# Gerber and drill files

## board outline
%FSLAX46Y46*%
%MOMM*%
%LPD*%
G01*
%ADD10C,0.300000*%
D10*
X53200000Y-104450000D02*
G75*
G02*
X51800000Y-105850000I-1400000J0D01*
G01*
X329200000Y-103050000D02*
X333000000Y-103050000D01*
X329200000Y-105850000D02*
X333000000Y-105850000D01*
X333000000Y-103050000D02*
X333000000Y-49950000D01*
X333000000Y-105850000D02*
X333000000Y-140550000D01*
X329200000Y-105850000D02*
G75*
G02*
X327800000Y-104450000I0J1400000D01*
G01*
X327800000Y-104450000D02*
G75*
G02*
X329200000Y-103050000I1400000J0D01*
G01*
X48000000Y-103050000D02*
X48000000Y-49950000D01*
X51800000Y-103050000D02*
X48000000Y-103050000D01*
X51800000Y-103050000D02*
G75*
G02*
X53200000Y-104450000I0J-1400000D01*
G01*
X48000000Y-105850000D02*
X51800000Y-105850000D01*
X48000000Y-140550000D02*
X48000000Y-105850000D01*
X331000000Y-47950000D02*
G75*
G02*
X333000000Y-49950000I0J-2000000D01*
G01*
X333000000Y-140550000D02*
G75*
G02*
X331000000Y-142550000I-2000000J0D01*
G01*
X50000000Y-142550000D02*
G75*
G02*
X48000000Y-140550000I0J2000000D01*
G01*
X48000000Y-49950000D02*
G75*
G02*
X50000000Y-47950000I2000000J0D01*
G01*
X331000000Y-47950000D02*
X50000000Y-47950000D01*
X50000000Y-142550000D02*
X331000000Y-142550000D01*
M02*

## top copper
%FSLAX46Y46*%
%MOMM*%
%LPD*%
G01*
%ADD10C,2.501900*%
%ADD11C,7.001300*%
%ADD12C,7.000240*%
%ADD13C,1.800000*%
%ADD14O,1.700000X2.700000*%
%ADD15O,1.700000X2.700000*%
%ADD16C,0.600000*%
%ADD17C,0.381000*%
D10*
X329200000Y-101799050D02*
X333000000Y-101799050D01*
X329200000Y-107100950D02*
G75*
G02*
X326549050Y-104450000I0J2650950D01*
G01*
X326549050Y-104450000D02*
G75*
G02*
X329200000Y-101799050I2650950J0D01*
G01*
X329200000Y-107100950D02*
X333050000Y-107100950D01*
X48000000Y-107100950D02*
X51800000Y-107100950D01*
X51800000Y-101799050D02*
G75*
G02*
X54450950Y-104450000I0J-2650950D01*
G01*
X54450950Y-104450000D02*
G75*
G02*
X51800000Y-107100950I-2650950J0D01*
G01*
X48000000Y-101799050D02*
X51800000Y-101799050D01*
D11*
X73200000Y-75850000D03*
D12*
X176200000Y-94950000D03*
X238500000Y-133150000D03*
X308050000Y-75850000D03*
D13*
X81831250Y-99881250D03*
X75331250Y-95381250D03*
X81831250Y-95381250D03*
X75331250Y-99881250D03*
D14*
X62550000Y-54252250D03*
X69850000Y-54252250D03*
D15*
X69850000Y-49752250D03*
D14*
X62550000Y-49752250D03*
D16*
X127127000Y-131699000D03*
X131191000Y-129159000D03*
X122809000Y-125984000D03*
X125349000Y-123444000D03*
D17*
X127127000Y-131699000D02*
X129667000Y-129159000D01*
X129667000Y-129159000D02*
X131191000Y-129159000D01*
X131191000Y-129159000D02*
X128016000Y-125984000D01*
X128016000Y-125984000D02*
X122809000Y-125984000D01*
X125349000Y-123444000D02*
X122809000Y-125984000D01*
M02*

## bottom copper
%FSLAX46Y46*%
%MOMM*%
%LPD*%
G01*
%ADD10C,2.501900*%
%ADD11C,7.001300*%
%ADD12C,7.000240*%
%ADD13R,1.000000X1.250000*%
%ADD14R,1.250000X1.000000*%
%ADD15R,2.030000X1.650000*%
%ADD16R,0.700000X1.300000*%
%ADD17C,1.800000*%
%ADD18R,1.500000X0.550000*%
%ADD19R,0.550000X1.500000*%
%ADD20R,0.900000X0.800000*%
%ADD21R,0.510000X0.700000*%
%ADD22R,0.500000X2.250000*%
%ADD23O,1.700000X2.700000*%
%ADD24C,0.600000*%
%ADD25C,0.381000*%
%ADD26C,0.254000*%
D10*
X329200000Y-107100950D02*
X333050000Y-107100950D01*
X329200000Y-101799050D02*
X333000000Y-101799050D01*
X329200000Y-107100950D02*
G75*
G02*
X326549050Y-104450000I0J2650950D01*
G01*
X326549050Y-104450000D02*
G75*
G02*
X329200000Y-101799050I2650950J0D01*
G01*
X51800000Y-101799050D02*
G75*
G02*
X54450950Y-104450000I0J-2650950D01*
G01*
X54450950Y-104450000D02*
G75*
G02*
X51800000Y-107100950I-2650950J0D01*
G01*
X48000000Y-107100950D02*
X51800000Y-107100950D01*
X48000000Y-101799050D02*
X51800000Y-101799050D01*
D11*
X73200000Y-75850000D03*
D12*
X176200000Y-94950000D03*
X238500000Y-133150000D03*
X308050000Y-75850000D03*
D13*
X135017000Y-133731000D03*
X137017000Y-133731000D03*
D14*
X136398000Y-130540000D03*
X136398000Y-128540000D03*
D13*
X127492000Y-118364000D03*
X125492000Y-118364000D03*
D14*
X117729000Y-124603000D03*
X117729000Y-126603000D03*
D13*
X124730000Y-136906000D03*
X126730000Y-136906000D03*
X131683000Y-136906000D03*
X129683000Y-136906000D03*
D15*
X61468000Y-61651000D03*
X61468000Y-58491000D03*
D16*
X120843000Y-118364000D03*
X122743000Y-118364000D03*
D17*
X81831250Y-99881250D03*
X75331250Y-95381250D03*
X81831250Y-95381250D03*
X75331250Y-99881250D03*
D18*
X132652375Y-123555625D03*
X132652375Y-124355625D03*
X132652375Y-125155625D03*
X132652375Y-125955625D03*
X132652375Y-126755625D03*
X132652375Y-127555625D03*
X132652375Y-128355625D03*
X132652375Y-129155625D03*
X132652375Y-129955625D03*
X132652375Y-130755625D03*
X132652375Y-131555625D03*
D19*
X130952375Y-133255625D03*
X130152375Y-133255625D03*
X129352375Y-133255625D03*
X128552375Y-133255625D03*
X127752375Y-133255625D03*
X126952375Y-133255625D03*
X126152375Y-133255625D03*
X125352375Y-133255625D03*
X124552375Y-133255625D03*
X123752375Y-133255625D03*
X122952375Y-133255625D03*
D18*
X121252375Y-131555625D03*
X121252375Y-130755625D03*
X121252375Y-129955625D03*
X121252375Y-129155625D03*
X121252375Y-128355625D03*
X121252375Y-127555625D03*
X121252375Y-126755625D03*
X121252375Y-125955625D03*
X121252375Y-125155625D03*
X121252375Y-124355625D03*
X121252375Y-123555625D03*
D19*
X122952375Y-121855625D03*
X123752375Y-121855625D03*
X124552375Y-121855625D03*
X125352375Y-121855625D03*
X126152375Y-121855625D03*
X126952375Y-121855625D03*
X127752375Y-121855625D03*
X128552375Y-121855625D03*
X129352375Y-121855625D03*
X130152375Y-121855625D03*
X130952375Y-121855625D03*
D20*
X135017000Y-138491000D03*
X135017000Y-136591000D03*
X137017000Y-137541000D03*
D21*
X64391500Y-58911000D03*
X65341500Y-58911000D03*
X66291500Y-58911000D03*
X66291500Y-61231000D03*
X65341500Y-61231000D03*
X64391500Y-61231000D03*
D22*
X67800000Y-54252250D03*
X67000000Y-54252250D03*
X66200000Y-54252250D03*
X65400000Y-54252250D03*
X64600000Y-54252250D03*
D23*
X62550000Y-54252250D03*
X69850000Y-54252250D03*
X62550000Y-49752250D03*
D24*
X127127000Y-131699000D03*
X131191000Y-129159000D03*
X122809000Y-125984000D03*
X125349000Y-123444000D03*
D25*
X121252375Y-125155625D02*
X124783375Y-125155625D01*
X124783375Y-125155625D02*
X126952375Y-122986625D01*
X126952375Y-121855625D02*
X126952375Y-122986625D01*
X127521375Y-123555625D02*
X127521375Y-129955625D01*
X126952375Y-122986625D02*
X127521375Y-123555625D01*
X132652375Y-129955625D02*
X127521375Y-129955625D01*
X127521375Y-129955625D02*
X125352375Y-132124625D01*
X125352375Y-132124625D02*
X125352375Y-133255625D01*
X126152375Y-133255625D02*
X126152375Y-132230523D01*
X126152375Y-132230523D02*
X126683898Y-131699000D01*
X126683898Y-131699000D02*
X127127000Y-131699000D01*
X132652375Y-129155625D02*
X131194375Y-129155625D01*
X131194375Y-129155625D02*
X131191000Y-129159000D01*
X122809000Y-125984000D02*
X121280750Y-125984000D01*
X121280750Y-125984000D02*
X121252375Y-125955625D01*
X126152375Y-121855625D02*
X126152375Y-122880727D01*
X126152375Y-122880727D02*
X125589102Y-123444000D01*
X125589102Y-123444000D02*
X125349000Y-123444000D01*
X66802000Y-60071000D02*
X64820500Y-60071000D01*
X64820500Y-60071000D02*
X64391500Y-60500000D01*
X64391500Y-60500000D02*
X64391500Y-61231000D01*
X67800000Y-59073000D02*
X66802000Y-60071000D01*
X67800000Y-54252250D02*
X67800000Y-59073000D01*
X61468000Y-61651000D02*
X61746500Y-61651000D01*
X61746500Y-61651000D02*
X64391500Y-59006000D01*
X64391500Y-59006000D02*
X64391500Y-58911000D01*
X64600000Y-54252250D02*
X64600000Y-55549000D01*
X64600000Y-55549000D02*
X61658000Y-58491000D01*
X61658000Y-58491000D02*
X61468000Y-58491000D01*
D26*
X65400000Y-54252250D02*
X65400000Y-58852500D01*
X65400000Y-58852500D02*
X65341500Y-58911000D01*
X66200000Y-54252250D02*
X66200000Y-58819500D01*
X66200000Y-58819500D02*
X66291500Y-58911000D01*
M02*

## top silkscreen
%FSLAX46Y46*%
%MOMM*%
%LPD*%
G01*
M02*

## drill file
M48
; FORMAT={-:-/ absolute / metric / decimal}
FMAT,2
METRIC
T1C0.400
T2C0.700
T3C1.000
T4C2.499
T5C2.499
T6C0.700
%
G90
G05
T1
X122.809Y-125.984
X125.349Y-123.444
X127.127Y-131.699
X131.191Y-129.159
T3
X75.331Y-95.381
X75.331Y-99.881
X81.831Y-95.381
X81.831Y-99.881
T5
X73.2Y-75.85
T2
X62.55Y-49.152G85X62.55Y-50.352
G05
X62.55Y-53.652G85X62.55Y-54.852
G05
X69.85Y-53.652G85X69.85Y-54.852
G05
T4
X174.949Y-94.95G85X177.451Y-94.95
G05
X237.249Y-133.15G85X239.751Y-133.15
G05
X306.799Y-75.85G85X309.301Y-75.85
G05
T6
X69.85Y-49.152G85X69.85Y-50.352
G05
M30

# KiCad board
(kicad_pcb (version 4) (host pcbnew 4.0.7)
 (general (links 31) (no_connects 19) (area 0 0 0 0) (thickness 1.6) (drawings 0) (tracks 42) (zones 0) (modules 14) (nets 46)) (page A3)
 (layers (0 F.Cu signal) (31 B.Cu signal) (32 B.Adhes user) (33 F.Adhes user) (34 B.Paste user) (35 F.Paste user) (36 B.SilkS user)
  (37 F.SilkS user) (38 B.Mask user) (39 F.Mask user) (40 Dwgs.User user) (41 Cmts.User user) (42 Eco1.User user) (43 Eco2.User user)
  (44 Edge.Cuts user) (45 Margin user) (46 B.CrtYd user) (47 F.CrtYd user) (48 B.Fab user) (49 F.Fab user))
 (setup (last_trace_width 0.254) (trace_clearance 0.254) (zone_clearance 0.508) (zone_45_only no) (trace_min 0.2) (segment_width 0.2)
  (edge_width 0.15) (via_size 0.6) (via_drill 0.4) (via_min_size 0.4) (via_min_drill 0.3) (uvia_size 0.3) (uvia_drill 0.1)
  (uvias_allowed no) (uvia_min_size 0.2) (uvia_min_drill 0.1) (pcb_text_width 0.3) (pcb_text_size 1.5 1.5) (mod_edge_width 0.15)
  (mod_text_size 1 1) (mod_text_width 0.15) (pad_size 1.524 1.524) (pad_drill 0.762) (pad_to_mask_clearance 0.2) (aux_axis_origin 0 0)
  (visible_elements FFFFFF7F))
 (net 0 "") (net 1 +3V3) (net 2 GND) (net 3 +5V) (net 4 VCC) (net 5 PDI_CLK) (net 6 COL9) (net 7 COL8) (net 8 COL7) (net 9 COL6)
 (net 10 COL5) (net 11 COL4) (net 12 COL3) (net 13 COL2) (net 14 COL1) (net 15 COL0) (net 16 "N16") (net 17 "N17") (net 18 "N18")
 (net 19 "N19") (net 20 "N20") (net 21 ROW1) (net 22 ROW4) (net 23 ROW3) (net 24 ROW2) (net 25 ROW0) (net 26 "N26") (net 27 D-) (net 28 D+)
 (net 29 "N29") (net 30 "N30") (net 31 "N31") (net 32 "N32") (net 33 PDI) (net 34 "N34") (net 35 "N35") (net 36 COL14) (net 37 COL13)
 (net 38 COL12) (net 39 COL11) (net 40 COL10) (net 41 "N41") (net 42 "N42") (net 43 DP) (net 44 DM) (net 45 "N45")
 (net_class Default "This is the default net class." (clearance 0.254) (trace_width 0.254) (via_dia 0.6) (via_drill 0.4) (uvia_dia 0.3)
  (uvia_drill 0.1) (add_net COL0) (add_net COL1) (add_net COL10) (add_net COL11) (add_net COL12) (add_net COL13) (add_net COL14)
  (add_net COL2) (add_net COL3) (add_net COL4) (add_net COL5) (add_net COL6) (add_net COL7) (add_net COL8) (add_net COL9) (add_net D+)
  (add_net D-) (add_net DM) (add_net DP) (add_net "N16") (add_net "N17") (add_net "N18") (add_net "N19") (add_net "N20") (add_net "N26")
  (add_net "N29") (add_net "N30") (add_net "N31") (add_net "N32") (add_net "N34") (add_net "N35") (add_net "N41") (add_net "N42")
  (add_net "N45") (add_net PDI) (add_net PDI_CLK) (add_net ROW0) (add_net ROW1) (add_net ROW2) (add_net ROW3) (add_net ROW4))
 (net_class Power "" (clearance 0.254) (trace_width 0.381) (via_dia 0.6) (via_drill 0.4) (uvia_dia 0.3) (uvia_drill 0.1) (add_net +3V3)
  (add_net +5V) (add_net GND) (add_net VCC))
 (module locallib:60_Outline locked (layer F.Cu) (at 190.5 95.25)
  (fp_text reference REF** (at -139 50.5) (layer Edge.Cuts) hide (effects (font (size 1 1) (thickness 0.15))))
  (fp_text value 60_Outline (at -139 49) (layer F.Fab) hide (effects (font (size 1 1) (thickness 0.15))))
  (fp_line (start 138.7 11.85095) (end 142.55 11.85095) (layer B.Cu) (width 2.5019))
  (fp_line (start 138.7 6.54905) (end 142.5 6.54905) (layer F.Cu) (width 2.5019))
  (fp_arc (start 138.7 9.2) (end 136.04905 9.2) (angle -90) (layer F.Cu) (width 2.5019))
  (fp_arc (start 138.7 9.2) (end 138.7 6.54905) (angle -90) (layer F.Cu) (width 2.5019))
  (fp_line (start 138.7 6.54905) (end 142.5 6.54905) (layer B.Cu) (width 2.5019))
  (fp_line (start 138.7 11.85095) (end 142.55 11.85095) (layer F.Cu) (width 2.5019))
  (fp_arc (start 138.7 9.2) (end 136.04905 9.2) (angle -90) (layer B.Cu) (width 2.5019))
  (fp_arc (start 138.7 9.2) (end 138.7 6.54905) (angle -90) (layer B.Cu) (width 2.5019))
  (fp_arc (start -138.7 9.2) (end -138.7 6.54905) (angle 90) (layer B.Cu) (width 2.5019))
  (fp_arc (start -138.7 9.2) (end -136.04905 9.2) (angle 90) (layer B.Cu) (width 2.5019))
  (fp_line (start -142.5 11.85095) (end -138.7 11.85095) (layer F.Cu) (width 2.5019))
  (fp_line (start -142.5 11.85095) (end -138.7 11.85095) (layer B.Cu) (width 2.5019))
  (fp_arc (start -138.7 9.2) (end -138.7 6.54905) (angle 90) (layer F.Cu) (width 2.5019))
  (fp_arc (start -138.7 9.2) (end -136.04905 9.2) (angle 90) (layer F.Cu) (width 2.5019))
  (fp_arc (start -138.7 9.2) (end -137.3 9.2) (angle 90) (layer Edge.Cuts) (width 0.3))
  (fp_line (start -142.5 6.54905) (end -138.7 6.54905) (layer B.Cu) (width 2.5019))
  (fp_line (start -142.5 6.54905) (end -138.7 6.54905) (layer F.Cu) (width 2.5019))
  (fp_line (start 138.7 7.8) (end 142.5 7.8) (layer Edge.Cuts) (width 0.3))
  (fp_line (start 138.7 10.6) (end 142.5 10.6) (layer Edge.Cuts) (width 0.3))
  (fp_line (start 142.5 7.8) (end 142.5 -45.3) (layer Edge.Cuts) (width 0.3))
  (fp_line (start 142.5 10.6) (end 142.5 45.3) (layer Edge.Cuts) (width 0.3))
  (fp_arc (start 138.7 9.2) (end 137.3 9.2) (angle -90) (layer Edge.Cuts) (width 0.3))
  (fp_arc (start 138.7 9.2) (end 138.7 7.8) (angle -90) (layer Edge.Cuts) (width 0.3))
  (fp_line (start -142.5 7.8) (end -142.5 -45.3) (layer Edge.Cuts) (width 0.3))
  (fp_line (start -138.7 7.8) (end -142.5 7.8) (layer Edge.Cuts) (width 0.3))
  (fp_arc (start -138.7 9.2) (end -138.7 7.8) (angle 90) (layer Edge.Cuts) (width 0.3))
  (fp_line (start -142.5 10.6) (end -138.7 10.6) (layer Edge.Cuts) (width 0.3))
  (fp_line (start -142.5 45.3) (end -142.5 10.6) (layer Edge.Cuts) (width 0.3))
  (fp_arc (start 140.5 -45.3) (end 140.5 -47.3) (angle 90) (layer Edge.Cuts) (width 0.3))
  (fp_arc (start 140.5 45.3) (end 142.5 45.3) (angle 90) (layer Edge.Cuts) (width 0.3))
  (fp_arc (start -140.5 45.3) (end -140.5 47.3) (angle 90) (layer Edge.Cuts) (width 0.3))
  (fp_arc (start -140.5 -45.3) (end -142.5 -45.3) (angle 90) (layer Edge.Cuts) (width 0.3))
  (fp_line (start 140.5 -47.3) (end -140.5 -47.3) (layer Edge.Cuts) (width 0.3))
  (fp_line (start -140.5 47.3) (end 140.5 47.3) (layer Edge.Cuts) (width 0.3))
  (pad 1 thru_hole circle (at -117.3 -19.4) (size 7.0013 7.0013) (drill 2.4994) (layers *.Cu *.Mask))
  (pad 1 thru_hole circle (at -14.3 -0.3) (size 7.00024 7.00024) (drill oval 5.00126 2.49936) (layers *.Cu *.Mask))
  (pad 1 thru_hole circle (at 48 37.9) (size 7.00024 7.00024) (drill oval 5.00126 2.49936) (layers *.Cu *.Mask))
  (pad 1 thru_hole circle (at 117.55 -19.4) (size 7.00024 7.00024) (drill oval 5.00126 2.49936) (layers *.Cu *.Mask)))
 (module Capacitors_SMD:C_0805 (layer B.Cu) (at 136.017 133.731)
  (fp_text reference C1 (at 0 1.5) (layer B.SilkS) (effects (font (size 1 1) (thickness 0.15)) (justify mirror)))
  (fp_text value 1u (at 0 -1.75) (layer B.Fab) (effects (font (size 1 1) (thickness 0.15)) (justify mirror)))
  (pad 1 smd rect (at -1 0) (size 1 1.25) (layers B.Cu B.Paste B.Mask) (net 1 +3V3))
  (pad 2 smd rect (at 1 0) (size 1 1.25) (layers B.Cu B.Paste B.Mask) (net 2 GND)))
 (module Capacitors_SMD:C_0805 (layer B.Cu) (at 136.398 129.54 90)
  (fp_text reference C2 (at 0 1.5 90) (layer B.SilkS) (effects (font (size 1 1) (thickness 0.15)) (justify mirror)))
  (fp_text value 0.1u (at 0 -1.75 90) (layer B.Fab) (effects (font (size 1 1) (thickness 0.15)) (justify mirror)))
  (pad 1 smd rect (at -1 0 90) (size 1 1.25) (layers B.Cu B.Paste B.Mask) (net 1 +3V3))
  (pad 2 smd rect (at 1 0 90) (size 1 1.25) (layers B.Cu B.Paste B.Mask) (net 2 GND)))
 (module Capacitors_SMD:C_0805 (layer B.Cu) (at 126.492 118.364 180)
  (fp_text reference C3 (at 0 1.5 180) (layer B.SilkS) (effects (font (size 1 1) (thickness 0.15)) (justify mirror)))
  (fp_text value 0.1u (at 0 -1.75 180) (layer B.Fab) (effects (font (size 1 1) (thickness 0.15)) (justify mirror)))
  (pad 1 smd rect (at -1 0 180) (size 1 1.25) (layers B.Cu B.Paste B.Mask) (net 1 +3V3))
  (pad 2 smd rect (at 1 0 180) (size 1 1.25) (layers B.Cu B.Paste B.Mask) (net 2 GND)))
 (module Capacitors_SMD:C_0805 (layer B.Cu) (at 117.729 125.603 270)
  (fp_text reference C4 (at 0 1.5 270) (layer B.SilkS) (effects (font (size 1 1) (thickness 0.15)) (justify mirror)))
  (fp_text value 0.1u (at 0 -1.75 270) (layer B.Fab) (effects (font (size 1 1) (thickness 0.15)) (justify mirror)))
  (pad 1 smd rect (at -1 0 270) (size 1 1.25) (layers B.Cu B.Paste B.Mask) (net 1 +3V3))
  (pad 2 smd rect (at 1 0 270) (size 1 1.25) (layers B.Cu B.Paste B.Mask) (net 2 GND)))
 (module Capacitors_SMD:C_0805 (layer B.Cu) (at 125.73 136.906)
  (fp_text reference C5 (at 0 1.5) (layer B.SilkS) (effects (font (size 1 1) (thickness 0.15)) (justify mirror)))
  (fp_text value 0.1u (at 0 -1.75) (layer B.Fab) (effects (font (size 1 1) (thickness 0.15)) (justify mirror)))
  (pad 1 smd rect (at -1 0) (size 1 1.25) (layers B.Cu B.Paste B.Mask) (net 1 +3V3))
  (pad 2 smd rect (at 1 0) (size 1 1.25) (layers B.Cu B.Paste B.Mask) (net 2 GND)))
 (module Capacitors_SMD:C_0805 (layer B.Cu) (at 130.683 136.906 180)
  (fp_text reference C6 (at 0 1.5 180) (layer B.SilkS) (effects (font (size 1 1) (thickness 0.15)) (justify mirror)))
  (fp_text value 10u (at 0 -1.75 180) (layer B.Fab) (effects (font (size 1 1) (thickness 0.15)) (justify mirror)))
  (pad 1 smd rect (at -1 0 180) (size 1 1.25) (layers B.Cu B.Paste B.Mask) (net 1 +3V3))
  (pad 2 smd rect (at 1 0 180) (size 1 1.25) (layers B.Cu B.Paste B.Mask) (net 2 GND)))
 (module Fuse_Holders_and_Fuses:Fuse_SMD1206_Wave (layer B.Cu) (at 61.468 60.071 90)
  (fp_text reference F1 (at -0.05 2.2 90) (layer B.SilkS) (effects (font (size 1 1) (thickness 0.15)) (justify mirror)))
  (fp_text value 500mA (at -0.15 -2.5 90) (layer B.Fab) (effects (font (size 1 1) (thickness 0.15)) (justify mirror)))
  (pad 1 smd rect (at -1.58 0) (size 2.03 1.65) (layers B.Cu B.Paste B.Mask) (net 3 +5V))
  (pad 2 smd rect (at 1.58 0) (size 2.03 1.65) (layers B.Cu B.Paste B.Mask) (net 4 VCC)))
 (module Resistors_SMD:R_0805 (layer B.Cu) (at 121.793 118.364)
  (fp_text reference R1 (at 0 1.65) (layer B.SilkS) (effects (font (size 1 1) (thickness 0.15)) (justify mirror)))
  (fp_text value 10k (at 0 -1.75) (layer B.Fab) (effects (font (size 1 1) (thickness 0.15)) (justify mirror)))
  (pad 1 smd rect (at -0.95 0) (size 0.7 1.3) (layers B.Cu B.Paste B.Mask) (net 1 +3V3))
  (pad 2 smd rect (at 0.95 0) (size 0.7 1.3) (layers B.Cu B.Paste B.Mask) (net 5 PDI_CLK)))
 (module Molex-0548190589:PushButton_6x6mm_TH (layer B.Cu) (at 78.58125 97.63125)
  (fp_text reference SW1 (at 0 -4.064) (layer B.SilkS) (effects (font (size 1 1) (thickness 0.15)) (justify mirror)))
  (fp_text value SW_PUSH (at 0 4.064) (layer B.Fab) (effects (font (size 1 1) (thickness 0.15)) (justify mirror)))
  (pad 1 thru_hole circle (at 3.25 2.25) (size 1.8 1.8) (drill 1) (layers *.Cu *.Mask) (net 2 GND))
  (pad 2 thru_hole circle (at -3.25 -2.25) (size 1.8 1.8) (drill 1) (layers *.Cu *.Mask) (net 5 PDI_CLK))
  (pad 3 thru_hole circle (at 3.25 -2.25) (size 1.8 1.8) (drill 1) (layers *.Cu *.Mask))
  (pad 4 thru_hole circle (at -3.25 2.25) (size 1.8 1.8) (drill 1) (layers *.Cu *.Mask)))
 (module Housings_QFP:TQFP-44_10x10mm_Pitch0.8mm (layer B.Cu) (at 126.952375 127.555625 180)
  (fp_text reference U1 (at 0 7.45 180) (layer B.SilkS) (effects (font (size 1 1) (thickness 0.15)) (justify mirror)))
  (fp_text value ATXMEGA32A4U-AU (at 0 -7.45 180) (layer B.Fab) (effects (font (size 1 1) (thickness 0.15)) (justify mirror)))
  (pad 1 smd rect (at -5.7 4 180) (size 1.5 0.55) (layers B.Cu B.Paste B.Mask) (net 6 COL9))
  (pad 2 smd rect (at -5.7 3.2 180) (size 1.5 0.55) (layers B.Cu B.Paste B.Mask) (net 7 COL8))
  (pad 3 smd rect (at -5.7 2.4 180) (size 1.5 0.55) (layers B.Cu B.Paste B.Mask) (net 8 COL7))
  (pad 4 smd rect (at -5.7 1.6 180) (size 1.5 0.55) (layers B.Cu B.Paste B.Mask) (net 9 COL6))
  (pad 5 smd rect (at -5.7 0.8 180) (size 1.5 0.55) (layers B.Cu B.Paste B.Mask) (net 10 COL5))
  (pad 6 smd rect (at -5.7 0 180) (size 1.5 0.55) (layers B.Cu B.Paste B.Mask) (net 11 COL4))
  (pad 7 smd rect (at -5.7 -0.8 180) (size 1.5 0.55) (layers B.Cu B.Paste B.Mask) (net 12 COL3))
  (pad 8 smd rect (at -5.7 -1.6 180) (size 1.5 0.55) (layers B.Cu B.Paste B.Mask) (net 2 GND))
  (pad 9 smd rect (at -5.7 -2.4 180) (size 1.5 0.55) (layers B.Cu B.Paste B.Mask) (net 1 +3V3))
  (pad 10 smd rect (at -5.7 -3.2 180) (size 1.5 0.55) (layers B.Cu B.Paste B.Mask) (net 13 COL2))
  (pad 11 smd rect (at -5.7 -4 180) (size 1.5 0.55) (layers B.Cu B.Paste B.Mask) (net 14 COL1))
  (pad 12 smd rect (at -4 -5.7 90) (size 1.5 0.55) (layers B.Cu B.Paste B.Mask) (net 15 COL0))
  (pad 13 smd rect (at -3.2 -5.7 90) (size 1.5 0.55) (layers B.Cu B.Paste B.Mask) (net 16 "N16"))
  (pad 14 smd rect (at -2.4 -5.7 90) (size 1.5 0.55) (layers B.Cu B.Paste B.Mask) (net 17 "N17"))
  (pad 15 smd rect (at -1.6 -5.7 90) (size 1.5 0.55) (layers B.Cu B.Paste B.Mask) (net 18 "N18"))
  (pad 16 smd rect (at -0.8 -5.7 90) (size 1.5 0.55) (layers B.Cu B.Paste B.Mask) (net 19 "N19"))
  (pad 17 smd rect (at 0 -5.7 90) (size 1.5 0.55) (layers B.Cu B.Paste B.Mask) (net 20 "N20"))
  (pad 18 smd rect (at 0.8 -5.7 90) (size 1.5 0.55) (layers B.Cu B.Paste B.Mask) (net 2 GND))
  (pad 19 smd rect (at 1.6 -5.7 90) (size 1.5 0.55) (layers B.Cu B.Paste B.Mask) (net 1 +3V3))
  (pad 20 smd rect (at 2.4 -5.7 90) (size 1.5 0.55) (layers B.Cu B.Paste B.Mask) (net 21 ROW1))
  (pad 21 smd rect (at 3.2 -5.7 90) (size 1.5 0.55) (layers B.Cu B.Paste B.Mask) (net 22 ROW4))
  (pad 22 smd rect (at 4 -5.7 90) (size 1.5 0.55) (layers B.Cu B.Paste B.Mask) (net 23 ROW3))
  (pad 23 smd rect (at 5.7 -4 180) (size 1.5 0.55) (layers B.Cu B.Paste B.Mask) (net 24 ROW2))
  (pad 24 smd rect (at 5.7 -3.2 180) (size 1.5 0.55) (layers B.Cu B.Paste B.Mask) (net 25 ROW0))
  (pad 25 smd rect (at 5.7 -2.4 180) (size 1.5 0.55) (layers B.Cu B.Paste B.Mask) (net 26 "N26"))
  (pad 26 smd rect (at 5.7 -1.6 180) (size 1.5 0.55) (layers B.Cu B.Paste B.Mask) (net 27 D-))
  (pad 27 smd rect (at 5.7 -0.8 180) (size 1.5 0.55) (layers B.Cu B.Paste B.Mask) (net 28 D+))
  (pad 28 smd rect (at 5.7 0 180) (size 1.5 0.55) (layers B.Cu B.Paste B.Mask) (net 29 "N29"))
  (pad 29 smd rect (at 5.7 0.8 180) (size 1.5 0.55) (layers B.Cu B.Paste B.Mask) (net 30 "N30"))
  (pad 30 smd rect (at 5.7 1.6 180) (size 1.5 0.55) (layers B.Cu B.Paste B.Mask) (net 2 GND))
  (pad 31 smd rect (at 5.7 2.4 180) (size 1.5 0.55) (layers B.Cu B.Paste B.Mask) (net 1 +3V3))
  (pad 32 smd rect (at 5.7 3.2 180) (size 1.5 0.55) (layers B.Cu B.Paste B.Mask) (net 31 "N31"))
  (pad 33 smd rect (at 5.7 4 180) (size 1.5 0.55) (layers B.Cu B.Paste B.Mask) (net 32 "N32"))
  (pad 34 smd rect (at 4 5.7 90) (size 1.5 0.55) (layers B.Cu B.Paste B.Mask) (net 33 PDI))
  (pad 35 smd rect (at 3.2 5.7 90) (size 1.5 0.55) (layers B.Cu B.Paste B.Mask) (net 5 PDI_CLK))
  (pad 36 smd rect (at 2.4 5.7 90) (size 1.5 0.55) (layers B.Cu B.Paste B.Mask) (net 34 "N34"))
  (pad 37 smd rect (at 1.6 5.7 90) (size 1.5 0.55) (layers B.Cu B.Paste B.Mask) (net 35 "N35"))
  (pad 38 smd rect (at 0.8 5.7 90) (size 1.5 0.55) (layers B.Cu B.Paste B.Mask) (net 2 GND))
  (pad 39 smd rect (at 0 5.7 90) (size 1.5 0.55) (layers B.Cu B.Paste B.Mask) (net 1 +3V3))
  (pad 40 smd rect (at -0.8 5.7 90) (size 1.5 0.55) (layers B.Cu B.Paste B.Mask) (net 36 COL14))
  (pad 41 smd rect (at -1.6 5.7 90) (size 1.5 0.55) (layers B.Cu B.Paste B.Mask) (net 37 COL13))
  (pad 42 smd rect (at -2.4 5.7 90) (size 1.5 0.55) (layers B.Cu B.Paste B.Mask) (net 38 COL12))
  (pad 43 smd rect (at -3.2 5.7 90) (size 1.5 0.55) (layers B.Cu B.Paste B.Mask) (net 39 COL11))
  (pad 44 smd rect (at -4 5.7 90) (size 1.5 0.55) (layers B.Cu B.Paste B.Mask) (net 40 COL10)))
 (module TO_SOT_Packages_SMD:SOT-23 (layer B.Cu) (at 136.017 137.541)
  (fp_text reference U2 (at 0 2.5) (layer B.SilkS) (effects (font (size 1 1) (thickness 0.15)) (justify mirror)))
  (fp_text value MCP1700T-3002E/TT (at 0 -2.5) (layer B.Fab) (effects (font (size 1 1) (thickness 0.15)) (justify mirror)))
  (pad 1 smd rect (at -1 0.95) (size 0.9 0.8) (layers B.Cu B.Paste B.Mask) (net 2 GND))
  (pad 2 smd rect (at -1 -0.95) (size 0.9 0.8) (layers B.Cu B.Paste B.Mask) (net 1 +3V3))
  (pad 3 smd rect (at 1 0) (size 0.9 0.8) (layers B.Cu B.Paste B.Mask) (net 3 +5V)))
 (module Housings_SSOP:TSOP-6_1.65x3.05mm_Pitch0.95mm (layer B.Cu) (at 65.3415 60.071 270)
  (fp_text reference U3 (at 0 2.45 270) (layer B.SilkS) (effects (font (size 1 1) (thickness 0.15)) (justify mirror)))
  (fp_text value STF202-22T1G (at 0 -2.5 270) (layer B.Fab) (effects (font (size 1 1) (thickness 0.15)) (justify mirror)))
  (pad 1 smd rect (at -1.16 0.95 270) (size 0.7 0.51) (layers B.Cu B.Paste B.Mask) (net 3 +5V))
  (pad 2 smd rect (at -1.16 0 270) (size 0.7 0.51) (layers B.Cu B.Paste B.Mask) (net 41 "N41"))
  (pad 3 smd rect (at -1.16 -0.95 270) (size 0.7 0.51) (layers B.Cu B.Paste B.Mask) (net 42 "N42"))
  (pad 4 smd rect (at 1.16 -0.95 270) (size 0.7 0.51) (layers B.Cu B.Paste B.Mask) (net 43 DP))
  (pad 5 smd rect (at 1.16 0 270) (size 0.7 0.51) (layers B.Cu B.Paste B.Mask) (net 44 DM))
  (pad 6 smd rect (at 1.16 0.95 270) (size 0.7 0.51) (layers B.Cu B.Paste B.Mask) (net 2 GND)))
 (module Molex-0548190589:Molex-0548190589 (layer B.Cu) (at 66.2 49.75225 270)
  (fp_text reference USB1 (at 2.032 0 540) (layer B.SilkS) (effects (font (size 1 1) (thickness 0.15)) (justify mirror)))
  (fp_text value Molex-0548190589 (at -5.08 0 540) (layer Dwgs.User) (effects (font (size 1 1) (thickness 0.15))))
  (pad 1 smd rect (at 4.5 -1.6 270) (size 2.25 0.5) (layers B.Cu B.Paste B.Mask) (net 2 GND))
  (pad 2 smd rect (at 4.5 -0.8 270) (size 2.25 0.5) (layers B.Cu B.Paste B.Mask) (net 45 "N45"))
  (pad 3 smd rect (at 4.5 0 270) (size 2.25 0.5) (layers B.Cu B.Paste B.Mask) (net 42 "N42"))
  (pad 4 smd rect (at 4.5 0.8 270) (size 2.25 0.5) (layers B.Cu B.Paste B.Mask) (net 41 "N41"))
  (pad 5 smd rect (at 4.5 1.6 270) (size 2.25 0.5) (layers B.Cu B.Paste B.Mask) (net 4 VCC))
  (pad "" thru_hole oval (at 4.5 3.65 270) (size 2.7 1.7) (drill oval 1.9 0.7) (layers F.Cu F.Mask))
  (pad "" thru_hole oval (at 4.5 -3.65 270) (size 2.7 1.7) (drill oval 1.9 0.7) (layers F.Cu F.Mask))
  (pad "" np_thru_hole oval (at 0 -3.65 270) (size 2.7 1.7) (drill oval 1.9 0.7) (layers F.Cu F.Mask))
  (pad "" thru_hole oval (at 0 3.65 270) (size 2.7 1.7) (drill oval 1.9 0.7) (layers F.Cu F.Mask)))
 (segment (start 121.252375 125.155625) (end 124.783375 125.155625) (width 0.381) (layer B.Cu) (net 1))
 (segment (start 124.783375 125.155625) (end 126.952375 122.986625) (width 0.381) (layer B.Cu) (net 1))
 (segment (start 126.952375 121.855625) (end 126.952375 122.986625) (width 0.381) (layer B.Cu) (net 1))
 (segment (start 127.521375 123.555625) (end 127.521375 129.955625) (width 0.381) (layer B.Cu) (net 1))
 (segment (start 126.952375 122.986625) (end 127.521375 123.555625) (width 0.381) (layer B.Cu) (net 1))
 (segment (start 132.652375 129.955625) (end 127.521375 129.955625) (width 0.381) (layer B.Cu) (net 1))
 (segment (start 127.521375 129.955625) (end 125.352375 132.124625) (width 0.381) (layer B.Cu) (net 1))
 (segment (start 125.352375 132.124625) (end 125.352375 133.255625) (width 0.381) (layer B.Cu) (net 1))
 (segment (start 127.127 131.699) (end 129.667 129.159) (width 0.381) (layer F.Cu) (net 2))
 (segment (start 129.667 129.159) (end 131.191 129.159) (width 0.381) (layer F.Cu) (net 2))
 (segment (start 126.152375 133.255625) (end 126.152375 132.230523) (width 0.381) (layer B.Cu) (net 2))
 (segment (start 126.152375 132.230523) (end 126.683898 131.699) (width 0.381) (layer B.Cu) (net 2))
 (segment (start 126.683898 131.699) (end 127.127 131.699) (width 0.381) (layer B.Cu) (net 2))
 (via (at 127.127 131.699) (size 0.6) (drill 0.4) (layers F.Cu B.Cu) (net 2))
 (segment (start 131.191 129.159) (end 128.016 125.984) (width 0.381) (layer F.Cu) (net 2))
 (segment (start 128.016 125.984) (end 122.809 125.984) (width 0.381) (layer F.Cu) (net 2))
 (segment (start 132.652375 129.155625) (end 131.194375 129.155625) (width 0.381) (layer B.Cu) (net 2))
 (segment (start 131.194375 129.155625) (end 131.191 129.159) (width 0.381) (layer B.Cu) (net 2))
 (via (at 131.191 129.159) (size 0.6) (drill 0.4) (layers F.Cu B.Cu) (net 2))
 (segment (start 122.809 125.984) (end 121.28075 125.984) (width 0.381) (layer B.Cu) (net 2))
 (segment (start 121.28075 125.984) (end 121.252375 125.955625) (width 0.381) (layer B.Cu) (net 2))
 (segment (start 125.349 123.444) (end 122.809 125.984) (width 0.381) (layer F.Cu) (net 2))
 (via (at 122.809 125.984) (size 0.6) (drill 0.4) (layers F.Cu B.Cu) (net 2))
 (segment (start 126.152375 121.855625) (end 126.152375 122.880727) (width 0.381) (layer B.Cu) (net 2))
 (segment (start 126.152375 122.880727) (end 125.589102 123.444) (width 0.381) (layer B.Cu) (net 2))
 (segment (start 125.589102 123.444) (end 125.349 123.444) (width 0.381) (layer B.Cu) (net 2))
 (via (at 125.349 123.444) (size 0.6) (drill 0.4) (layers F.Cu B.Cu) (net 2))
 (segment (start 66.802 60.071) (end 64.8205 60.071) (width 0.381) (layer B.Cu) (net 2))
 (segment (start 64.8205 60.071) (end 64.3915 60.5) (width 0.381) (layer B.Cu) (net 2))
 (segment (start 64.3915 60.5) (end 64.3915 61.231) (width 0.381) (layer B.Cu) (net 2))
 (segment (start 67.8 59.073) (end 66.802 60.071) (width 0.381) (layer B.Cu) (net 2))
 (segment (start 67.8 54.25225) (end 67.8 59.073) (width 0.381) (layer B.Cu) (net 2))
 (segment (start 61.468 61.651) (end 61.7465 61.651) (width 0.381) (layer B.Cu) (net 3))
 (segment (start 61.7465 61.651) (end 64.3915 59.006) (width 0.381) (layer B.Cu) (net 3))
 (segment (start 64.3915 59.006) (end 64.3915 58.911) (width 0.381) (layer B.Cu) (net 3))
 (segment (start 64.6 54.25225) (end 64.6 55.549) (width 0.381) (layer B.Cu) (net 4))
 (segment (start 64.6 55.549) (end 61.658 58.491) (width 0.381) (layer B.Cu) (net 4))
 (segment (start 61.658 58.491) (end 61.468 58.491) (width 0.381) (layer B.Cu) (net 4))
 (segment (start 65.4 54.25225) (end 65.4 58.8525) (width 0.254) (layer B.Cu) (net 41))
 (segment (start 65.4 58.8525) (end 65.3415 58.911) (width 0.254) (layer B.Cu) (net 41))
 (segment (start 66.2 54.25225) (end 66.2 58.8195) (width 0.254) (layer B.Cu) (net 42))
 (segment (start 66.2 58.8195) (end 66.2915 58.911) (width 0.254) (layer B.Cu) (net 42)))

